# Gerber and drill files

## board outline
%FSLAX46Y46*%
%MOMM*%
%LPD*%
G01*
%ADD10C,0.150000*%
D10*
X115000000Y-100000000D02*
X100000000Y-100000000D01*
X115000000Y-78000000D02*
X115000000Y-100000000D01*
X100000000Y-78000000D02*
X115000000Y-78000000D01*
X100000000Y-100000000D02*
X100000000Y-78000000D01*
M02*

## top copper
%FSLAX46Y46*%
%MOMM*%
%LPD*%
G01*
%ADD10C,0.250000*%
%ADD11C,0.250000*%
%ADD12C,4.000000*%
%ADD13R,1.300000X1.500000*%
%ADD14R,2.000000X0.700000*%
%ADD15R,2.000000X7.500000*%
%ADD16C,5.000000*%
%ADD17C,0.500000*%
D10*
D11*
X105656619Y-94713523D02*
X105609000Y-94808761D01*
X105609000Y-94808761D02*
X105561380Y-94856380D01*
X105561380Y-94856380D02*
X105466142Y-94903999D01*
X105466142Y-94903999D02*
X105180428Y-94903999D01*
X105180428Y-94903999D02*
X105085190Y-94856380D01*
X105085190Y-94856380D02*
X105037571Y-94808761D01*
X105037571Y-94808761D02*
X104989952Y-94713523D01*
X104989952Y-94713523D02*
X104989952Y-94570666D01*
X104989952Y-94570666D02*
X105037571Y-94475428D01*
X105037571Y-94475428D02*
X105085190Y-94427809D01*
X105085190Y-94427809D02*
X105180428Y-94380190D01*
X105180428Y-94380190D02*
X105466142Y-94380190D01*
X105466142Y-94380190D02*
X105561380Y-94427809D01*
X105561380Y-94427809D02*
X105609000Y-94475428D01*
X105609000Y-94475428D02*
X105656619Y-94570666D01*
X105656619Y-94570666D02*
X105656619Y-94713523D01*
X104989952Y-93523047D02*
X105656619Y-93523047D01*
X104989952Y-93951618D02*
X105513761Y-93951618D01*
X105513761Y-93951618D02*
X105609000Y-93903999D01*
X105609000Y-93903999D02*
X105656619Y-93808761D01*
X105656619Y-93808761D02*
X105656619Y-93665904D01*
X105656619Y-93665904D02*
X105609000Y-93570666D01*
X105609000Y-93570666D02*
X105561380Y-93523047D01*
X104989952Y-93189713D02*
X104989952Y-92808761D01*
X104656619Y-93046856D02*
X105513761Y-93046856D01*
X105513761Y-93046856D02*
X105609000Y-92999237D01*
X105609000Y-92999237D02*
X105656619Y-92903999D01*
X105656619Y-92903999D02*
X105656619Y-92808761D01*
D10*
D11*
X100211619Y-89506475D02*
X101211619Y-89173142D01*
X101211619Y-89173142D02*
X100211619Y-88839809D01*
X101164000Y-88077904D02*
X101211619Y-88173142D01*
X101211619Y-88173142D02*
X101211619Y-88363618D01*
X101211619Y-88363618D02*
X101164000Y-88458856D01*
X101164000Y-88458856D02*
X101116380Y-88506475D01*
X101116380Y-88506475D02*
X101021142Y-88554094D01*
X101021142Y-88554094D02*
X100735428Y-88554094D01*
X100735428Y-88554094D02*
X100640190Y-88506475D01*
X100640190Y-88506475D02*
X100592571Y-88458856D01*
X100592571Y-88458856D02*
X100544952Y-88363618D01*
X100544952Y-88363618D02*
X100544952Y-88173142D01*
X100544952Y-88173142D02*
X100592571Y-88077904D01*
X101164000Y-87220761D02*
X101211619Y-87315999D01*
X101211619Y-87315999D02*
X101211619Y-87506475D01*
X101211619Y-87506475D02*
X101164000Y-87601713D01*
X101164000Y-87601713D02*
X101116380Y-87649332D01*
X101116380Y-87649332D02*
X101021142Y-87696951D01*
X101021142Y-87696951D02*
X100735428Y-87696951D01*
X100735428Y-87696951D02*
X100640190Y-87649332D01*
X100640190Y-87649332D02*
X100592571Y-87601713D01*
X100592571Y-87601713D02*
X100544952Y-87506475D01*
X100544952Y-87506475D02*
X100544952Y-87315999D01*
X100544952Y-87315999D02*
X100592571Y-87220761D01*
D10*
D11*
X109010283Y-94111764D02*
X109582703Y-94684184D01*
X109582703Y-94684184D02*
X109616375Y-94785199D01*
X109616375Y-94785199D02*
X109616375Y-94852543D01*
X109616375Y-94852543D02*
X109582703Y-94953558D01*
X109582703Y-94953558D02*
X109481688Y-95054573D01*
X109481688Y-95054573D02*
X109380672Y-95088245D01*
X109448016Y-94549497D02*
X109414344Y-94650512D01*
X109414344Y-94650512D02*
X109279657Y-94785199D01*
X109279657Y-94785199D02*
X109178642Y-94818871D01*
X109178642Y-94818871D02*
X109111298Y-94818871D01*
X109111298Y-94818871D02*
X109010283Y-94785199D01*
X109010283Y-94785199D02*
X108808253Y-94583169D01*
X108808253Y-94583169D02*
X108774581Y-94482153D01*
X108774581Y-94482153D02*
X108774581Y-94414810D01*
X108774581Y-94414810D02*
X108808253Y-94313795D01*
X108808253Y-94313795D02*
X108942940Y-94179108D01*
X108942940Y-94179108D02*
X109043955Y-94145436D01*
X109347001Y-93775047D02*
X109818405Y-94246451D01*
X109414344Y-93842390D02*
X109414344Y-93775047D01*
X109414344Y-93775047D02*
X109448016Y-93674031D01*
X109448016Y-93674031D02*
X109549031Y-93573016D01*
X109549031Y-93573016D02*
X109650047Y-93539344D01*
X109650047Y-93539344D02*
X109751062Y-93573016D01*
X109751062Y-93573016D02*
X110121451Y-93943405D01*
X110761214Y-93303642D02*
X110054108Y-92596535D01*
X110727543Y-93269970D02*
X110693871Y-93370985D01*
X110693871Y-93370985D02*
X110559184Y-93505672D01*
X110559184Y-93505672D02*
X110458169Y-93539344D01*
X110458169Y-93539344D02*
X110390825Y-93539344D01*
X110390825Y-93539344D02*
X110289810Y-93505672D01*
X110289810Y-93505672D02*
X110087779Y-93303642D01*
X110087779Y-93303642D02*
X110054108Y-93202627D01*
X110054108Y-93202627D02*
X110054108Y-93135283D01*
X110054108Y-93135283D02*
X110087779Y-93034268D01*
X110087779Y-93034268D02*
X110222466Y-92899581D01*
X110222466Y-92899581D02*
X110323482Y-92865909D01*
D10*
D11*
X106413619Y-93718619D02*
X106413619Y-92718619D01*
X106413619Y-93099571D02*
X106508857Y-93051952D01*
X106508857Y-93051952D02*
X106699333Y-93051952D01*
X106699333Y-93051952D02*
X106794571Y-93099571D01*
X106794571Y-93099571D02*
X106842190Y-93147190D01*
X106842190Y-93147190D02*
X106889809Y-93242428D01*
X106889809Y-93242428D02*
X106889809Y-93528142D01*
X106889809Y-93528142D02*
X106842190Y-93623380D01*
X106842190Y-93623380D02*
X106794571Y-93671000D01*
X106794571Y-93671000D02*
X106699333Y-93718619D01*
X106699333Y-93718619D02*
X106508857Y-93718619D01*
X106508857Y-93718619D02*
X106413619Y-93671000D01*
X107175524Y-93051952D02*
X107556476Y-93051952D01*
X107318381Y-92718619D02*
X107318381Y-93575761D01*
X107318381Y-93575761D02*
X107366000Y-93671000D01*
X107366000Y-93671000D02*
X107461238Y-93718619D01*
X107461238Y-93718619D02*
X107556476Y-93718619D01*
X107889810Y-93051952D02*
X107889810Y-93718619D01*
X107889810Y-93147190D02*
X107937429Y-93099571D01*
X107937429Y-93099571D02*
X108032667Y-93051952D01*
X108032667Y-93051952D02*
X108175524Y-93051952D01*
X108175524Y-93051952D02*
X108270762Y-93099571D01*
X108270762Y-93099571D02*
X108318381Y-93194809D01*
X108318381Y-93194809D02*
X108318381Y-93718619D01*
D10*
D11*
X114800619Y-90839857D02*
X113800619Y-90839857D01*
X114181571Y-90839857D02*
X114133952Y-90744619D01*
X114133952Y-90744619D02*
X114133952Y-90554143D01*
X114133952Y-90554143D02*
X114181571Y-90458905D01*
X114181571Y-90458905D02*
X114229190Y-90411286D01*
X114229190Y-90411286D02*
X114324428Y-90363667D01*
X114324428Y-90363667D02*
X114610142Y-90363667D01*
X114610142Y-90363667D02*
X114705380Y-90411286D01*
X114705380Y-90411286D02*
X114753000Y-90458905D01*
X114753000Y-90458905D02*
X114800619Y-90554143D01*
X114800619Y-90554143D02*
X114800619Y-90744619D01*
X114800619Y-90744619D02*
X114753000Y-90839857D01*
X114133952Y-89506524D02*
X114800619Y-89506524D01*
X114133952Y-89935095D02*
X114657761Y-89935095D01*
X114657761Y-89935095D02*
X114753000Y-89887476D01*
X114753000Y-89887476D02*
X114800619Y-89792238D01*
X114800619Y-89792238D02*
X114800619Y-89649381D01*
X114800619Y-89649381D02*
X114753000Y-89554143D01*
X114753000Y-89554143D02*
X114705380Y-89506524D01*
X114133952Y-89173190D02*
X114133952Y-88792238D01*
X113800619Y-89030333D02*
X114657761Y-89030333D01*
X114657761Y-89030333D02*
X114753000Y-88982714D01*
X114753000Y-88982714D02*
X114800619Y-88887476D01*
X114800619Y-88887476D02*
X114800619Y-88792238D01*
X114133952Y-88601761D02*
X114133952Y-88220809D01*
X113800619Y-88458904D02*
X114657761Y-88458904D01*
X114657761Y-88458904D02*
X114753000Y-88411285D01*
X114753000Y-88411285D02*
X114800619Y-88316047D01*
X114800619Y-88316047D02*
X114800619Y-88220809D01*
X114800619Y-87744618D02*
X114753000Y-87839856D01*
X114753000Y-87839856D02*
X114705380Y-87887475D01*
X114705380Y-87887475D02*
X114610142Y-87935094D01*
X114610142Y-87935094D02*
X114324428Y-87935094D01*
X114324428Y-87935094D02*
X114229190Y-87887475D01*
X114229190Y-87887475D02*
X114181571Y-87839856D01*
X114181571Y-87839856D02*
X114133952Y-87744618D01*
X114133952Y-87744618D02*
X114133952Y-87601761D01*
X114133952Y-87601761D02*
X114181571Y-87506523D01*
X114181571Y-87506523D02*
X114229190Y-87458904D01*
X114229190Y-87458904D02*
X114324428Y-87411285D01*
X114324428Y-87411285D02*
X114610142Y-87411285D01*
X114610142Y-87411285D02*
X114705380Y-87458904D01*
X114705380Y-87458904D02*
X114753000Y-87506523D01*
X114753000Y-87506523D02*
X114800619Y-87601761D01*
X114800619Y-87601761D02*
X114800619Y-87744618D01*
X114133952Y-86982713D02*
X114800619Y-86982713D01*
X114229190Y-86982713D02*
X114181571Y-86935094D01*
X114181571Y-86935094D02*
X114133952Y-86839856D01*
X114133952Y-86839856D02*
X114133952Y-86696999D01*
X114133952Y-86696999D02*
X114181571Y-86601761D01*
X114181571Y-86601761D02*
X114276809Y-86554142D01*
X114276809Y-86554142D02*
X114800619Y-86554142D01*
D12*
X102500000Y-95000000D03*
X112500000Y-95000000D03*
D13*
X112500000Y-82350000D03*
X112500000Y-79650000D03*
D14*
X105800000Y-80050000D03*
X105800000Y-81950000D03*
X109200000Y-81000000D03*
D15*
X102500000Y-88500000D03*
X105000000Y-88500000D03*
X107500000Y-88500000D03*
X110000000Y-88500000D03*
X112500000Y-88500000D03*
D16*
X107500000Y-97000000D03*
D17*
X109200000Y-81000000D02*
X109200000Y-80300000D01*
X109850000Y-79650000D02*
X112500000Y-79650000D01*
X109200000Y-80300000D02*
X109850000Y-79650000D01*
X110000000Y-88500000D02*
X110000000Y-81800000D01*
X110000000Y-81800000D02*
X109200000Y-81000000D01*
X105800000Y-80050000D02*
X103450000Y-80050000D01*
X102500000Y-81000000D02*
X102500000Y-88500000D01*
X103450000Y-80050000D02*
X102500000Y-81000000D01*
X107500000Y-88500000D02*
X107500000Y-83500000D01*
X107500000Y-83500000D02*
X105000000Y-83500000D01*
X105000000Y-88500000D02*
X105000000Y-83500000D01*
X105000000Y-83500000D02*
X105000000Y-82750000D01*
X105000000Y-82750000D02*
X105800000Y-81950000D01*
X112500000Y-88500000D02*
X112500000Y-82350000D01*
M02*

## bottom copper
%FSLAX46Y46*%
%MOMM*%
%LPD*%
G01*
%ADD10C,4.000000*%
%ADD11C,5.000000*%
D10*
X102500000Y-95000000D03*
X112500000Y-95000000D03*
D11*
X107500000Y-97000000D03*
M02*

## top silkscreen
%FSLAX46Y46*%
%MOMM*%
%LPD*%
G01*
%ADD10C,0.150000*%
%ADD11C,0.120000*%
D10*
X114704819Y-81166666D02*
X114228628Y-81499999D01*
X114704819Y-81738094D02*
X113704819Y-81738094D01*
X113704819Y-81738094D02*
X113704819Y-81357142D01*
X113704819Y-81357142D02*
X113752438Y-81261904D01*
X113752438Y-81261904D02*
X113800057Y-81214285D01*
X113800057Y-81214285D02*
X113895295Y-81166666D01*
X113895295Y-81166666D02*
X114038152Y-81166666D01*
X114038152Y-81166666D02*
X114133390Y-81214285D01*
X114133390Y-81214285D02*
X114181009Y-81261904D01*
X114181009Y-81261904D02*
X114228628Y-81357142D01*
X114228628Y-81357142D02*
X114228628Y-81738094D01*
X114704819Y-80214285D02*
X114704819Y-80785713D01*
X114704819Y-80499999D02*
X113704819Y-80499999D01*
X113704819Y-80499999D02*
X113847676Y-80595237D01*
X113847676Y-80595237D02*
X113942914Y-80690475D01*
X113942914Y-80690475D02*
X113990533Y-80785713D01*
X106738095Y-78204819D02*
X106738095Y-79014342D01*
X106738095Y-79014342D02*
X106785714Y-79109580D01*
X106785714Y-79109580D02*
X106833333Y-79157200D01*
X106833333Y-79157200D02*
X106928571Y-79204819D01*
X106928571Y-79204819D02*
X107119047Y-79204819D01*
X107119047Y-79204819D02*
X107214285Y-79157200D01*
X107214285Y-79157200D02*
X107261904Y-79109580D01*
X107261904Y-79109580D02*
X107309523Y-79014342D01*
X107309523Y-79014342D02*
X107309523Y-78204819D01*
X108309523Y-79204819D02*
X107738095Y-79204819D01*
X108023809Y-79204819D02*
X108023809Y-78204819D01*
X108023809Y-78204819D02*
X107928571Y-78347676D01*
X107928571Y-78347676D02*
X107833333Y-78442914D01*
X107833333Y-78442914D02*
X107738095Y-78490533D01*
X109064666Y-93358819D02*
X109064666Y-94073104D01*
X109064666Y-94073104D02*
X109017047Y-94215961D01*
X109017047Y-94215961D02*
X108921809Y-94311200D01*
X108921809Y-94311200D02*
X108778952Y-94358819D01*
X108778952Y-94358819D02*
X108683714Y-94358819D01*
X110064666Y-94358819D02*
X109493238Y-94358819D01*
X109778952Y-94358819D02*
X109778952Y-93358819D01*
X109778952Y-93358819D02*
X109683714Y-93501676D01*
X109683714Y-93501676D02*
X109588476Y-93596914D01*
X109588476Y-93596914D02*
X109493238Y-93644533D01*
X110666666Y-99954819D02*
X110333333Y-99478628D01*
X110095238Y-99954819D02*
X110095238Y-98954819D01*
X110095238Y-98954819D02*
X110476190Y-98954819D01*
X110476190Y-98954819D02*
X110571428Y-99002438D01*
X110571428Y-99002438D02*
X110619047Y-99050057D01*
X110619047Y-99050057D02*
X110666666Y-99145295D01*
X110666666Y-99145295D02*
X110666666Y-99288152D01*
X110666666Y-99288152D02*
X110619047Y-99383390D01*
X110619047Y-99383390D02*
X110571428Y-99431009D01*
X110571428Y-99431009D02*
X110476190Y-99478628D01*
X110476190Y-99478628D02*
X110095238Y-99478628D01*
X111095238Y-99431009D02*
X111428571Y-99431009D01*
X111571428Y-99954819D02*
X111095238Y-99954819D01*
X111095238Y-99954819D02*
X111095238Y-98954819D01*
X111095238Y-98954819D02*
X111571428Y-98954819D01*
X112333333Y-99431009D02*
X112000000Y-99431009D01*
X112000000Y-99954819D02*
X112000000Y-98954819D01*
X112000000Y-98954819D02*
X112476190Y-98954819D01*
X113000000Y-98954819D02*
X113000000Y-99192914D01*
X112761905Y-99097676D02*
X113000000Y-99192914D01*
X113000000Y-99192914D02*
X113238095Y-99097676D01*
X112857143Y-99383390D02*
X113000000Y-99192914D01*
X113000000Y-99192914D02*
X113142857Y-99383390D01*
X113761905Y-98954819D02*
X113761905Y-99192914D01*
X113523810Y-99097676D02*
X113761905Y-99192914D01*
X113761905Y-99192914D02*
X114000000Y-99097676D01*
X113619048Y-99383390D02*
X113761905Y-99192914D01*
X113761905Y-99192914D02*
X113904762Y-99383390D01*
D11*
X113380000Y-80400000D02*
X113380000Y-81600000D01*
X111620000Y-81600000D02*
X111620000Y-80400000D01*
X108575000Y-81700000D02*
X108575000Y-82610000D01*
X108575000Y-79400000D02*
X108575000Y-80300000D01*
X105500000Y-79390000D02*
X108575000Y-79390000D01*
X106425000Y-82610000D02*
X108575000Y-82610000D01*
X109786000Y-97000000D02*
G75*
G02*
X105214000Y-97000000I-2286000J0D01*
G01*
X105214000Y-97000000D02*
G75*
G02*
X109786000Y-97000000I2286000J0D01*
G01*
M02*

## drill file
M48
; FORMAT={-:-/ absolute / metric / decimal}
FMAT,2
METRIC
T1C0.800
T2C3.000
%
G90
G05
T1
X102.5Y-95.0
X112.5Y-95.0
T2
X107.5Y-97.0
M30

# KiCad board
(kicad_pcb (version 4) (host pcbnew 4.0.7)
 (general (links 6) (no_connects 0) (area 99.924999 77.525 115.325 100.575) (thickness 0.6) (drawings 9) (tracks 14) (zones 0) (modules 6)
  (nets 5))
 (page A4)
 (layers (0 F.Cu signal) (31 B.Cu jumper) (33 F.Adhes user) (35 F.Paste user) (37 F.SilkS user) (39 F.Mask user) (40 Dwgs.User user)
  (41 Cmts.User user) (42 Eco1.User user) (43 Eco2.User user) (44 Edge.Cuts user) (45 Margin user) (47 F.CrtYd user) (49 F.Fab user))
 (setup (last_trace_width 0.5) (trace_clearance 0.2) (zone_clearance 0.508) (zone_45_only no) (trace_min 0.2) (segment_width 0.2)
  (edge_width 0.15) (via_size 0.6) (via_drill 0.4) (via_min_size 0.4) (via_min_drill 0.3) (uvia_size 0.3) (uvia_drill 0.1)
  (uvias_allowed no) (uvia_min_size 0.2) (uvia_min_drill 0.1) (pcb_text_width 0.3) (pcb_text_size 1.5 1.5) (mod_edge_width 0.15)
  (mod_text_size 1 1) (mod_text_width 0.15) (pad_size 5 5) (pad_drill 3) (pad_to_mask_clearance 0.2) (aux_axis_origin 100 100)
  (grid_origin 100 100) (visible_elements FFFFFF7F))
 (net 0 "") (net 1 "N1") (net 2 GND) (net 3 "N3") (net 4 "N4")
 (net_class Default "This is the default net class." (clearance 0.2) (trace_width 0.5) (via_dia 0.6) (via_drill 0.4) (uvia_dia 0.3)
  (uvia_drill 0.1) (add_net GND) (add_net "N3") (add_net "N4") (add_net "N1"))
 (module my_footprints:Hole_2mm (layer F.Cu) (at 103.5 95)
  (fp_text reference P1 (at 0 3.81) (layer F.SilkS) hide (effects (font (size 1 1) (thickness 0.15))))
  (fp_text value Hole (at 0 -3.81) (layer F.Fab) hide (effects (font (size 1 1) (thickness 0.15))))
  (pad "" np_thru_hole circle (at -1 0) (size 4 4) (drill 0.8) (layers *.Cu *.Mask)))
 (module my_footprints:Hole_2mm (layer F.Cu) (at 111.5 95)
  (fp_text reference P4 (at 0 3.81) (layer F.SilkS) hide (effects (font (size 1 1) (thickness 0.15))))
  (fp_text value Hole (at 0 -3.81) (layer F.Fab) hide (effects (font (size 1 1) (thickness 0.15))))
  (pad "" np_thru_hole circle (at 1 0) (size 4 4) (drill 0.8) (layers *.Cu *.Mask)))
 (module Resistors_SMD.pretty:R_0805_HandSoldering (layer F.Cu) (at 112.5 81 90)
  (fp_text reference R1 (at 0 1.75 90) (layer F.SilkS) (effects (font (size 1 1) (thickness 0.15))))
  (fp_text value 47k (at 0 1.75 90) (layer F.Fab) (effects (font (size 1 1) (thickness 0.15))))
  (fp_line (start 0.6 0.88) (end -0.6 0.88) (layer F.SilkS) (width 0.12))
  (fp_line (start -0.6 -0.88) (end 0.6 -0.88) (layer F.SilkS) (width 0.12))
  (pad 1 smd rect (at -1.35 0 90) (size 1.5 1.3) (layers F.Cu F.Paste F.Mask) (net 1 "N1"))
  (pad 2 smd rect (at 1.35 0 90) (size 1.5 1.3) (layers F.Cu F.Paste F.Mask) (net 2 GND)))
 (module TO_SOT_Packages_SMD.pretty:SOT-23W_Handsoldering (layer F.Cu) (at 107.5 81)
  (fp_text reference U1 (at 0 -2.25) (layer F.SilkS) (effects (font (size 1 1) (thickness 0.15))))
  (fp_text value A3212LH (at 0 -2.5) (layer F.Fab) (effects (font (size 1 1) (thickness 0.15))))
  (fp_line (start 1.075 0.7) (end 1.075 1.61) (layer F.SilkS) (width 0.12))
  (fp_line (start 1.075 -1.6) (end 1.075 -0.7) (layer F.SilkS) (width 0.12))
  (fp_line (start -2 -1.61) (end 1.075 -1.61) (layer F.SilkS) (width 0.12))
  (fp_line (start -1.075 1.61) (end 1.075 1.61) (layer F.SilkS) (width 0.12))
  (pad 1 smd rect (at -1.7 -0.95) (size 2 0.7) (layers F.Cu F.Paste F.Mask) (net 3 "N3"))
  (pad 2 smd rect (at -1.7 0.95) (size 2 0.7) (layers F.Cu F.Paste F.Mask) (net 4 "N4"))
  (pad 3 smd rect (at 1.7 0) (size 2 0.7) (layers F.Cu F.Paste F.Mask) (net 2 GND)))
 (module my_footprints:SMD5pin (layer F.Cu) (at 107.5 88.5)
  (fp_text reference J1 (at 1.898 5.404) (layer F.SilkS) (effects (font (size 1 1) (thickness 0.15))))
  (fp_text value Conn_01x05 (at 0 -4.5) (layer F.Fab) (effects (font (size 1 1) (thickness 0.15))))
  (pad 1 smd rect (at -5 0) (size 2 7.5) (layers F.Cu F.Paste F.Mask) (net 3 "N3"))
  (pad 2 smd rect (at -2.5 0) (size 2 7.5) (layers F.Cu F.Paste F.Mask) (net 4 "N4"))
  (pad 3 smd rect (at 0 0) (size 2 7.5) (layers F.Cu F.Paste F.Mask) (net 4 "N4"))
  (pad 4 smd rect (at 2.5 0) (size 2 7.5) (layers F.Cu F.Paste F.Mask) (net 2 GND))
  (pad 5 smd rect (at 5 0) (size 2 7.5) (layers F.Cu F.Paste F.Mask) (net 1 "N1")))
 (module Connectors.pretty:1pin (layer F.Cu) (at 107.5 97)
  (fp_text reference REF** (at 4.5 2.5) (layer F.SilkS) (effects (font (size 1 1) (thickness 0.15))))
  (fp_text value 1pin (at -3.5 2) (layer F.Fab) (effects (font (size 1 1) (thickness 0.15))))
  (fp_circle (center 0 0) (end 0 -2.286) (layer F.SilkS) (width 0.12))
  (pad "" np_thru_hole circle (at 0 0) (size 5 5) (drill 3) (layers *.Cu *.Mask)))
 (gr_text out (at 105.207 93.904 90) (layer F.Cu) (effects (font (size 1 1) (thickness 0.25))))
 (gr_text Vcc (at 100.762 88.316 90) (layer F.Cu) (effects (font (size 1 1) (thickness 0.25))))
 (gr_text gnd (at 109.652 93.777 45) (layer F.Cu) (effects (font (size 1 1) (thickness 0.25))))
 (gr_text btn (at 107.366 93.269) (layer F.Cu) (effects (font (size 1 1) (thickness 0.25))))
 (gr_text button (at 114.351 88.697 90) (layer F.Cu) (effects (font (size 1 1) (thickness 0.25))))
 (gr_line (start 115 100) (end 100 100) (angle 90) (layer Edge.Cuts) (width 0.15))
 (gr_line (start 115 78) (end 115 100) (angle 90) (layer Edge.Cuts) (width 0.15))
 (gr_line (start 100 78) (end 115 78) (angle 90) (layer Edge.Cuts) (width 0.15))
 (gr_line (start 100 100) (end 100 78) (angle 90) (layer Edge.Cuts) (width 0.15))
 (segment (start 109.2 81) (end 109.2 80.3) (width 0.5) (layer F.Cu) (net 2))
 (segment (start 109.85 79.65) (end 112.5 79.65) (width 0.5) (layer F.Cu) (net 2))
 (segment (start 109.2 80.3) (end 109.85 79.65) (width 0.5) (layer F.Cu) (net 2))
 (segment (start 110 88.5) (end 110 81.8) (width 0.5) (layer F.Cu) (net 2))
 (segment (start 110 81.8) (end 109.2 81) (width 0.5) (layer F.Cu) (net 2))
 (segment (start 105.8 80.05) (end 103.45 80.05) (width 0.5) (layer F.Cu) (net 3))
 (segment (start 102.5 81) (end 102.5 88.5) (width 0.5) (layer F.Cu) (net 3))
 (segment (start 103.45 80.05) (end 102.5 81) (width 0.5) (layer F.Cu) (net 3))
 (segment (start 107.5 88.5) (end 107.5 83.5) (width 0.5) (layer F.Cu) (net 4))
 (segment (start 107.5 83.5) (end 105 83.5) (width 0.5) (layer F.Cu) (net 4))
 (segment (start 105 88.5) (end 105 83.5) (width 0.5) (layer F.Cu) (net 4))
 (segment (start 105 83.5) (end 105 82.75) (width 0.5) (layer F.Cu) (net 4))
 (segment (start 105 82.75) (end 105.8 81.95) (width 0.5) (layer F.Cu) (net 4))
 (segment (start 112.5 88.5) (end 112.5 82.35) (width 0.5) (layer F.Cu) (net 1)))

